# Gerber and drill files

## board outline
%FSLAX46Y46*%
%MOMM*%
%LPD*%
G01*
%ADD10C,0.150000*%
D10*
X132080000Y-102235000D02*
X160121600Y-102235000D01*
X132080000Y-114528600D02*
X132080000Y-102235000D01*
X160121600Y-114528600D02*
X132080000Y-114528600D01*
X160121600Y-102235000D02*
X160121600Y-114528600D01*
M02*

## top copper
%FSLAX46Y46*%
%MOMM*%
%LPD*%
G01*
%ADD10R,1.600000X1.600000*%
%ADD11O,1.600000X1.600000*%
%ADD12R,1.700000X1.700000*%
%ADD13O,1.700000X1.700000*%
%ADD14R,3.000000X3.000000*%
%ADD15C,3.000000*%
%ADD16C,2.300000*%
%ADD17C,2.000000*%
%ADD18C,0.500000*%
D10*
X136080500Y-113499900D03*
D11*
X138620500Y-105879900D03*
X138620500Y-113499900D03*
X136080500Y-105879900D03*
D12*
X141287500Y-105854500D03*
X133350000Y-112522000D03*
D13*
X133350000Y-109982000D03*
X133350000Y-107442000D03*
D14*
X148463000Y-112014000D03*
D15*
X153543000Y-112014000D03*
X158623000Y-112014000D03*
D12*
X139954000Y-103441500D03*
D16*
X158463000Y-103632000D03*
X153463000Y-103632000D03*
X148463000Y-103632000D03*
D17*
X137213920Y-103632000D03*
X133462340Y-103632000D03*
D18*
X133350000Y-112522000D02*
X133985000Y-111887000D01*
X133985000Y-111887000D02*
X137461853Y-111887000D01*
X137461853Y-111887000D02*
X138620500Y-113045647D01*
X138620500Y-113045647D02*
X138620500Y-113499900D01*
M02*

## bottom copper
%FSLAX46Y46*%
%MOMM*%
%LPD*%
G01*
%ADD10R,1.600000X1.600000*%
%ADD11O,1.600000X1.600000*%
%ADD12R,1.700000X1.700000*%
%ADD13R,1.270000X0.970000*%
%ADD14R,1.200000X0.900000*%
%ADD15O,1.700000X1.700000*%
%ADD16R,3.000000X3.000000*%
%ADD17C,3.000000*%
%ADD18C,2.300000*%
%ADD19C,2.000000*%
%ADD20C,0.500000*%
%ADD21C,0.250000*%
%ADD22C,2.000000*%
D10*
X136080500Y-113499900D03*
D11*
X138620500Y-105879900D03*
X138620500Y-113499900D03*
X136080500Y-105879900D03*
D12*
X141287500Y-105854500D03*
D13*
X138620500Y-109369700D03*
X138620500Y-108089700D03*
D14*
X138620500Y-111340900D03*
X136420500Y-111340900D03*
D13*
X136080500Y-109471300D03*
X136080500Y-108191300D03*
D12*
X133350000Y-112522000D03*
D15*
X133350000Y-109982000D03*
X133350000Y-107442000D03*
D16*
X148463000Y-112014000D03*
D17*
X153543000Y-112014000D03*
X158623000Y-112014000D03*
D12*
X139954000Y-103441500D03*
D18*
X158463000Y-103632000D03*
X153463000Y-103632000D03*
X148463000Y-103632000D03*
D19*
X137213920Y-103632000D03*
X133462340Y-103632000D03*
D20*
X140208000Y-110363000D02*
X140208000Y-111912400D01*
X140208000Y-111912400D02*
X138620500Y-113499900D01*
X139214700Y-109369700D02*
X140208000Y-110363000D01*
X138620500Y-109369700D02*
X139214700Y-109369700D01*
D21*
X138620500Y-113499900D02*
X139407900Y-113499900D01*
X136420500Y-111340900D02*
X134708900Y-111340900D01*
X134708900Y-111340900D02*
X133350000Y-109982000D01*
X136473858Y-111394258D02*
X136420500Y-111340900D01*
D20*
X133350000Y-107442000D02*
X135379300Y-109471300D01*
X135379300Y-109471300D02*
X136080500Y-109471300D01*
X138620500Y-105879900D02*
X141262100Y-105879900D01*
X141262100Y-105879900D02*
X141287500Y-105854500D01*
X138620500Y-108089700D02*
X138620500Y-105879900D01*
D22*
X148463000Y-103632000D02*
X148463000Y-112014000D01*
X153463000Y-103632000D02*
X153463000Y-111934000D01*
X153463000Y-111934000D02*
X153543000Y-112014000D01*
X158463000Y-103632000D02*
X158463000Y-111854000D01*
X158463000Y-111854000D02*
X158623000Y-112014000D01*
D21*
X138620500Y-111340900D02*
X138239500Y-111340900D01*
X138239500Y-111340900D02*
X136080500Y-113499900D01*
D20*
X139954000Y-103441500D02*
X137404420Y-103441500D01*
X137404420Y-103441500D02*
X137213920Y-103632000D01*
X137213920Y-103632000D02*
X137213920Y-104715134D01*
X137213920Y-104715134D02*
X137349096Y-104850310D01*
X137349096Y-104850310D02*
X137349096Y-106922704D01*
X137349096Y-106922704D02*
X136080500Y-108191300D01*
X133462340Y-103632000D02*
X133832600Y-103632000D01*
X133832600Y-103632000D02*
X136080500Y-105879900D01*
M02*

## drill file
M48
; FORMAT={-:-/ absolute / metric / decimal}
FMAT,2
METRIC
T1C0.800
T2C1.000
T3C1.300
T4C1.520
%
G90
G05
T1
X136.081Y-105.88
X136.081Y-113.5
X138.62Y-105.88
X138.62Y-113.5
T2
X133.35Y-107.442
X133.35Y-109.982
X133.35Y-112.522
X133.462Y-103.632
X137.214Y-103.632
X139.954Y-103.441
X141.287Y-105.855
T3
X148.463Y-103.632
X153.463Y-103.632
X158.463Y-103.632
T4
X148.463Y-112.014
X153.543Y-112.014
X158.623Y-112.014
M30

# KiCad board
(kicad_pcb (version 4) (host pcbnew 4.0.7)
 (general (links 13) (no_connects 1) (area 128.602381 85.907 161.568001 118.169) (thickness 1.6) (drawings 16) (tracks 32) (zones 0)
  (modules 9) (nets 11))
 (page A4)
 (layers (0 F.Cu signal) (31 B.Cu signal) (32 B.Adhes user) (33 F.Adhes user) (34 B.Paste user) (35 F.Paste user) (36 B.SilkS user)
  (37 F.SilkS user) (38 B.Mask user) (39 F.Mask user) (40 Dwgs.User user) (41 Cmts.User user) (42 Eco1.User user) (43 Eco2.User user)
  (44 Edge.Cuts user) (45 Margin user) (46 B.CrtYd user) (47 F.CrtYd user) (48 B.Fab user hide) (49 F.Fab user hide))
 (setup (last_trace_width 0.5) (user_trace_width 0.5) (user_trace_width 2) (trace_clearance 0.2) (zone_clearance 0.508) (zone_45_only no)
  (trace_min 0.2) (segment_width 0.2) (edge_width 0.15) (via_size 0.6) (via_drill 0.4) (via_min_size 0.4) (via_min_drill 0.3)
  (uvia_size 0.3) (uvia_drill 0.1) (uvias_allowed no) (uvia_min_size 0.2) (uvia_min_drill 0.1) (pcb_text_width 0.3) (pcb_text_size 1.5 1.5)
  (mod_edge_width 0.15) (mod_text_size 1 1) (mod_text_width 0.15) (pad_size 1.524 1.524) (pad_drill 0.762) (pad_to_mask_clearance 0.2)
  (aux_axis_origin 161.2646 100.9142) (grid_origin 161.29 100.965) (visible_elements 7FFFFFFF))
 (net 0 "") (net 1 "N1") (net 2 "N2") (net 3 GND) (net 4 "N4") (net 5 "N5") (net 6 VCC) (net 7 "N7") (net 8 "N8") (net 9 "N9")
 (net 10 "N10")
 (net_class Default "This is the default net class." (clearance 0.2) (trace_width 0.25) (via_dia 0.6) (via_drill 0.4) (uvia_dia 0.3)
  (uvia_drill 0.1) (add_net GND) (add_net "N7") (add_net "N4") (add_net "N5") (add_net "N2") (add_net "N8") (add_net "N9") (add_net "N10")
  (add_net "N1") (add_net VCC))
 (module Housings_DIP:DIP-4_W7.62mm (layer F.Cu) (at 136.0805 113.4999 90)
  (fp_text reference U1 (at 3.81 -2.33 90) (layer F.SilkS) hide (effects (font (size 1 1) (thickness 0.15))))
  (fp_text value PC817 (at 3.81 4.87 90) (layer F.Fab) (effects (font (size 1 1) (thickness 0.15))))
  (pad 1 thru_hole rect (at 0 0 90) (size 1.6 1.6) (drill 0.8) (layers *.Cu *.Mask) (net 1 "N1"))
  (pad 3 thru_hole oval (at 7.62 2.54 90) (size 1.6 1.6) (drill 0.8) (layers *.Cu *.Mask) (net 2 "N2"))
  (pad 2 thru_hole oval (at 0 2.54 90) (size 1.6 1.6) (drill 0.8) (layers *.Cu *.Mask) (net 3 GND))
  (pad 4 thru_hole oval (at 7.62 0 90) (size 1.6 1.6) (drill 0.8) (layers *.Cu *.Mask) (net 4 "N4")))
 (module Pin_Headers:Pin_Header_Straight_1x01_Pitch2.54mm (layer F.Cu) (at 141.2875 105.8545 90)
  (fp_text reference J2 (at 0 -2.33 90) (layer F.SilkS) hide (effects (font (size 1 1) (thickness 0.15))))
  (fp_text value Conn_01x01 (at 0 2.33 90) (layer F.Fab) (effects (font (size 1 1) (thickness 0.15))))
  (pad 1 thru_hole rect (at 0 0 90) (size 1.7 1.7) (drill 1) (layers *.Cu *.Mask) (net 2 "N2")))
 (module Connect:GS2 (layer B.Cu) (at 138.6205 108.7297)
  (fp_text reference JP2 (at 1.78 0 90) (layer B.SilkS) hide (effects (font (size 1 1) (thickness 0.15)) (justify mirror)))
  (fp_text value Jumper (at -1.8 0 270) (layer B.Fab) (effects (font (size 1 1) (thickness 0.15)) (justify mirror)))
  (pad 1 smd rect (at 0 0.64) (size 1.27 0.97) (layers B.Cu B.Paste B.Mask) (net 3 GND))
  (pad 2 smd rect (at 0 -0.64) (size 1.27 0.97) (layers B.Cu B.Paste B.Mask) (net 2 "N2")))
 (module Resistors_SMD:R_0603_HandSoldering (layer B.Cu) (at 137.5205 111.3409 180)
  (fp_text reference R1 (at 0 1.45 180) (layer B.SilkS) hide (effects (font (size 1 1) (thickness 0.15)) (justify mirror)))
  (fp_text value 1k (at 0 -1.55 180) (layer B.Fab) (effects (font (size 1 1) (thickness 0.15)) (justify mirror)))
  (pad 1 smd rect (at -1.1 0 180) (size 1.2 0.9) (layers B.Cu B.Paste B.Mask) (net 1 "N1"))
  (pad 2 smd rect (at 1.1 0 180) (size 1.2 0.9) (layers B.Cu B.Paste B.Mask) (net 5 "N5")))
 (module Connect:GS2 (layer B.Cu) (at 136.0805 108.8313)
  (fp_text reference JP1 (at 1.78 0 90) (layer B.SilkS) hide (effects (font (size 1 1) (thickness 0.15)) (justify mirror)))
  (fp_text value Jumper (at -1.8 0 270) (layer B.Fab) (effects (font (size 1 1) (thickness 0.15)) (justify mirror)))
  (pad 1 smd rect (at 0 0.64) (size 1.27 0.97) (layers B.Cu B.Paste B.Mask) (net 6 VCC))
  (pad 2 smd rect (at 0 -0.64) (size 1.27 0.97) (layers B.Cu B.Paste B.Mask) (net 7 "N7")))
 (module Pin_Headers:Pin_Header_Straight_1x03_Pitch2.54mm (layer F.Cu) (at 133.35 112.522 180)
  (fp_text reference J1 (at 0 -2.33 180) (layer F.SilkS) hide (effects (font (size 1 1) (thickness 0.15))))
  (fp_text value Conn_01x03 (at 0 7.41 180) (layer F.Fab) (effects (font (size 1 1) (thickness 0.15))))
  (pad 1 thru_hole rect (at 0 0 180) (size 1.7 1.7) (drill 1) (layers *.Cu *.Mask) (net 3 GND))
  (pad 2 thru_hole oval (at 0 2.54 180) (size 1.7 1.7) (drill 1) (layers *.Cu *.Mask) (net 5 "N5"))
  (pad 3 thru_hole oval (at 0 5.08 180) (size 1.7 1.7) (drill 1) (layers *.Cu *.Mask) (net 6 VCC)))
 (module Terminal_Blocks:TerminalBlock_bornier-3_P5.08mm (layer F.Cu) (at 148.463 112.014)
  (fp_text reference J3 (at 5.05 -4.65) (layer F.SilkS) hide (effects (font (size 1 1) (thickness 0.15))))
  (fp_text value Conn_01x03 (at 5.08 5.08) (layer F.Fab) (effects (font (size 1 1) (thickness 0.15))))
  (pad 1 thru_hole rect (at 0 0) (size 3 3) (drill 1.52) (layers *.Cu *.Mask) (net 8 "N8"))
  (pad 2 thru_hole circle (at 5.08 0) (size 3 3) (drill 1.52) (layers *.Cu *.Mask) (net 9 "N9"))
  (pad 3 thru_hole circle (at 10.16 0) (size 3 3) (drill 1.52) (layers *.Cu *.Mask) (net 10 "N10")))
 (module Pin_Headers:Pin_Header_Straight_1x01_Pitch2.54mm (layer F.Cu) (at 139.954 103.4415)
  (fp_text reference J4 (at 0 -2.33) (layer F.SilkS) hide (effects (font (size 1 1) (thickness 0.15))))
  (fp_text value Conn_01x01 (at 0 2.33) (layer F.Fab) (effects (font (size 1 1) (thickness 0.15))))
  (pad 1 thru_hole rect (at 0 0) (size 1.7 1.7) (drill 1) (layers *.Cu *.Mask) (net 7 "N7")))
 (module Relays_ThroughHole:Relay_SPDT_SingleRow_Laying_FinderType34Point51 (layer F.Cu) (at 137.21392 103.632)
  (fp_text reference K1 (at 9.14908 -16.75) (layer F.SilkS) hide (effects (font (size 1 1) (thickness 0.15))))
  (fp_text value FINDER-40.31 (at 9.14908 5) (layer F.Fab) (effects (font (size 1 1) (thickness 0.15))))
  (pad 14 thru_hole circle (at 21.24908 0) (size 2.3 2.3) (drill 1.3) (layers *.Cu *.Mask) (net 10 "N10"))
  (pad 11 thru_hole circle (at 16.24908 0) (size 2.3 2.3) (drill 1.3) (layers *.Cu *.Mask) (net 9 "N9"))
  (pad 12 thru_hole circle (at 11.24908 0) (size 2.3 2.3) (drill 1.3) (layers *.Cu *.Mask) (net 8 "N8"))
  (pad A1 thru_hole circle (at 0 0) (size 2 2) (drill 1) (layers *.Cu *.Mask) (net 7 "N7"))
  (pad A2 thru_hole circle (at -3.75158 0) (size 2 2) (drill 1) (layers *.Cu *.Mask) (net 4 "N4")))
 (gr_line (start 132.08 102.235) (end 160.1216 102.235) (layer Edge.Cuts) (width 0.15))
 (gr_line (start 132.08 114.5286) (end 132.08 102.235) (layer Edge.Cuts) (width 0.15))
 (gr_line (start 160.1216 114.5286) (end 132.08 114.5286) (layer Edge.Cuts) (width 0.15))
 (gr_line (start 160.1216 102.235) (end 160.1216 114.5286) (layer Edge.Cuts) (width 0.15))
 (segment (start 140.208 110.363) (end 140.208 111.9124) (width 0.5) (layer B.Cu) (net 3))
 (segment (start 140.208 111.9124) (end 138.6205 113.4999) (width 0.5) (layer B.Cu) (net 3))
 (segment (start 139.2147 109.3697) (end 140.208 110.363) (width 0.5) (layer B.Cu) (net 3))
 (segment (start 138.6205 109.3697) (end 139.2147 109.3697) (width 0.5) (layer B.Cu) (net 3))
 (segment (start 133.35 112.522) (end 133.985 111.887) (width 0.5) (layer F.Cu) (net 3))
 (segment (start 133.985 111.887) (end 137.461853 111.887) (width 0.5) (layer F.Cu) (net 3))
 (segment (start 137.461853 111.887) (end 138.6205 113.045647) (width 0.5) (layer F.Cu) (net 3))
 (segment (start 138.6205 113.045647) (end 138.6205 113.4999) (width 0.5) (layer F.Cu) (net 3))
 (segment (start 138.6205 113.4999) (end 139.4079 113.4999) (width 0.25) (layer B.Cu) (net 3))
 (segment (start 136.4205 111.3409) (end 134.7089 111.3409) (width 0.25) (layer B.Cu) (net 5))
 (segment (start 134.7089 111.3409) (end 133.35 109.982) (width 0.25) (layer B.Cu) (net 5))
 (segment (start 136.473858 111.394258) (end 136.4205 111.3409) (width 0.25) (layer B.Cu) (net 5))
 (segment (start 133.35 107.442) (end 135.3793 109.4713) (width 0.5) (layer B.Cu) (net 6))
 (segment (start 135.3793 109.4713) (end 136.0805 109.4713) (width 0.5) (layer B.Cu) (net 6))
 (segment (start 138.6205 105.8799) (end 141.2621 105.8799) (width 0.5) (layer B.Cu) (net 2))
 (segment (start 141.2621 105.8799) (end 141.2875 105.8545) (width 0.5) (layer B.Cu) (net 2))
 (segment (start 138.6205 108.0897) (end 138.6205 105.8799) (width 0.5) (layer B.Cu) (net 2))
 (segment (start 148.463 103.632) (end 148.463 112.014) (width 2) (layer B.Cu) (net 8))
 (segment (start 153.463 103.632) (end 153.463 111.934) (width 2) (layer B.Cu) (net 9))
 (segment (start 153.463 111.934) (end 153.543 112.014) (width 2) (layer B.Cu) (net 9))
 (segment (start 158.463 103.632) (end 158.463 111.854) (width 2) (layer B.Cu) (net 10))
 (segment (start 158.463 111.854) (end 158.623 112.014) (width 2) (layer B.Cu) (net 10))
 (segment (start 138.6205 111.3409) (end 138.2395 111.3409) (width 0.25) (layer B.Cu) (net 1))
 (segment (start 138.2395 111.3409) (end 136.0805 113.4999) (width 0.25) (layer B.Cu) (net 1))
 (segment (start 139.954 103.4415) (end 137.40442 103.4415) (width 0.5) (layer B.Cu) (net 7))
 (segment (start 137.40442 103.4415) (end 137.21392 103.632) (width 0.5) (layer B.Cu) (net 7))
 (segment (start 137.21392 103.632) (end 137.21392 104.715134) (width 0.5) (layer B.Cu) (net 7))
 (segment (start 137.21392 104.715134) (end 137.349096 104.85031) (width 0.5) (layer B.Cu) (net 7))
 (segment (start 137.349096 104.85031) (end 137.349096 106.922704) (width 0.5) (layer B.Cu) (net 7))
 (segment (start 137.349096 106.922704) (end 136.0805 108.1913) (width 0.5) (layer B.Cu) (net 7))
 (segment (start 133.46234 103.632) (end 133.8326 103.632) (width 0.5) (layer B.Cu) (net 4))
 (segment (start 133.8326 103.632) (end 136.0805 105.8799) (width 0.5) (layer B.Cu) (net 4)))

